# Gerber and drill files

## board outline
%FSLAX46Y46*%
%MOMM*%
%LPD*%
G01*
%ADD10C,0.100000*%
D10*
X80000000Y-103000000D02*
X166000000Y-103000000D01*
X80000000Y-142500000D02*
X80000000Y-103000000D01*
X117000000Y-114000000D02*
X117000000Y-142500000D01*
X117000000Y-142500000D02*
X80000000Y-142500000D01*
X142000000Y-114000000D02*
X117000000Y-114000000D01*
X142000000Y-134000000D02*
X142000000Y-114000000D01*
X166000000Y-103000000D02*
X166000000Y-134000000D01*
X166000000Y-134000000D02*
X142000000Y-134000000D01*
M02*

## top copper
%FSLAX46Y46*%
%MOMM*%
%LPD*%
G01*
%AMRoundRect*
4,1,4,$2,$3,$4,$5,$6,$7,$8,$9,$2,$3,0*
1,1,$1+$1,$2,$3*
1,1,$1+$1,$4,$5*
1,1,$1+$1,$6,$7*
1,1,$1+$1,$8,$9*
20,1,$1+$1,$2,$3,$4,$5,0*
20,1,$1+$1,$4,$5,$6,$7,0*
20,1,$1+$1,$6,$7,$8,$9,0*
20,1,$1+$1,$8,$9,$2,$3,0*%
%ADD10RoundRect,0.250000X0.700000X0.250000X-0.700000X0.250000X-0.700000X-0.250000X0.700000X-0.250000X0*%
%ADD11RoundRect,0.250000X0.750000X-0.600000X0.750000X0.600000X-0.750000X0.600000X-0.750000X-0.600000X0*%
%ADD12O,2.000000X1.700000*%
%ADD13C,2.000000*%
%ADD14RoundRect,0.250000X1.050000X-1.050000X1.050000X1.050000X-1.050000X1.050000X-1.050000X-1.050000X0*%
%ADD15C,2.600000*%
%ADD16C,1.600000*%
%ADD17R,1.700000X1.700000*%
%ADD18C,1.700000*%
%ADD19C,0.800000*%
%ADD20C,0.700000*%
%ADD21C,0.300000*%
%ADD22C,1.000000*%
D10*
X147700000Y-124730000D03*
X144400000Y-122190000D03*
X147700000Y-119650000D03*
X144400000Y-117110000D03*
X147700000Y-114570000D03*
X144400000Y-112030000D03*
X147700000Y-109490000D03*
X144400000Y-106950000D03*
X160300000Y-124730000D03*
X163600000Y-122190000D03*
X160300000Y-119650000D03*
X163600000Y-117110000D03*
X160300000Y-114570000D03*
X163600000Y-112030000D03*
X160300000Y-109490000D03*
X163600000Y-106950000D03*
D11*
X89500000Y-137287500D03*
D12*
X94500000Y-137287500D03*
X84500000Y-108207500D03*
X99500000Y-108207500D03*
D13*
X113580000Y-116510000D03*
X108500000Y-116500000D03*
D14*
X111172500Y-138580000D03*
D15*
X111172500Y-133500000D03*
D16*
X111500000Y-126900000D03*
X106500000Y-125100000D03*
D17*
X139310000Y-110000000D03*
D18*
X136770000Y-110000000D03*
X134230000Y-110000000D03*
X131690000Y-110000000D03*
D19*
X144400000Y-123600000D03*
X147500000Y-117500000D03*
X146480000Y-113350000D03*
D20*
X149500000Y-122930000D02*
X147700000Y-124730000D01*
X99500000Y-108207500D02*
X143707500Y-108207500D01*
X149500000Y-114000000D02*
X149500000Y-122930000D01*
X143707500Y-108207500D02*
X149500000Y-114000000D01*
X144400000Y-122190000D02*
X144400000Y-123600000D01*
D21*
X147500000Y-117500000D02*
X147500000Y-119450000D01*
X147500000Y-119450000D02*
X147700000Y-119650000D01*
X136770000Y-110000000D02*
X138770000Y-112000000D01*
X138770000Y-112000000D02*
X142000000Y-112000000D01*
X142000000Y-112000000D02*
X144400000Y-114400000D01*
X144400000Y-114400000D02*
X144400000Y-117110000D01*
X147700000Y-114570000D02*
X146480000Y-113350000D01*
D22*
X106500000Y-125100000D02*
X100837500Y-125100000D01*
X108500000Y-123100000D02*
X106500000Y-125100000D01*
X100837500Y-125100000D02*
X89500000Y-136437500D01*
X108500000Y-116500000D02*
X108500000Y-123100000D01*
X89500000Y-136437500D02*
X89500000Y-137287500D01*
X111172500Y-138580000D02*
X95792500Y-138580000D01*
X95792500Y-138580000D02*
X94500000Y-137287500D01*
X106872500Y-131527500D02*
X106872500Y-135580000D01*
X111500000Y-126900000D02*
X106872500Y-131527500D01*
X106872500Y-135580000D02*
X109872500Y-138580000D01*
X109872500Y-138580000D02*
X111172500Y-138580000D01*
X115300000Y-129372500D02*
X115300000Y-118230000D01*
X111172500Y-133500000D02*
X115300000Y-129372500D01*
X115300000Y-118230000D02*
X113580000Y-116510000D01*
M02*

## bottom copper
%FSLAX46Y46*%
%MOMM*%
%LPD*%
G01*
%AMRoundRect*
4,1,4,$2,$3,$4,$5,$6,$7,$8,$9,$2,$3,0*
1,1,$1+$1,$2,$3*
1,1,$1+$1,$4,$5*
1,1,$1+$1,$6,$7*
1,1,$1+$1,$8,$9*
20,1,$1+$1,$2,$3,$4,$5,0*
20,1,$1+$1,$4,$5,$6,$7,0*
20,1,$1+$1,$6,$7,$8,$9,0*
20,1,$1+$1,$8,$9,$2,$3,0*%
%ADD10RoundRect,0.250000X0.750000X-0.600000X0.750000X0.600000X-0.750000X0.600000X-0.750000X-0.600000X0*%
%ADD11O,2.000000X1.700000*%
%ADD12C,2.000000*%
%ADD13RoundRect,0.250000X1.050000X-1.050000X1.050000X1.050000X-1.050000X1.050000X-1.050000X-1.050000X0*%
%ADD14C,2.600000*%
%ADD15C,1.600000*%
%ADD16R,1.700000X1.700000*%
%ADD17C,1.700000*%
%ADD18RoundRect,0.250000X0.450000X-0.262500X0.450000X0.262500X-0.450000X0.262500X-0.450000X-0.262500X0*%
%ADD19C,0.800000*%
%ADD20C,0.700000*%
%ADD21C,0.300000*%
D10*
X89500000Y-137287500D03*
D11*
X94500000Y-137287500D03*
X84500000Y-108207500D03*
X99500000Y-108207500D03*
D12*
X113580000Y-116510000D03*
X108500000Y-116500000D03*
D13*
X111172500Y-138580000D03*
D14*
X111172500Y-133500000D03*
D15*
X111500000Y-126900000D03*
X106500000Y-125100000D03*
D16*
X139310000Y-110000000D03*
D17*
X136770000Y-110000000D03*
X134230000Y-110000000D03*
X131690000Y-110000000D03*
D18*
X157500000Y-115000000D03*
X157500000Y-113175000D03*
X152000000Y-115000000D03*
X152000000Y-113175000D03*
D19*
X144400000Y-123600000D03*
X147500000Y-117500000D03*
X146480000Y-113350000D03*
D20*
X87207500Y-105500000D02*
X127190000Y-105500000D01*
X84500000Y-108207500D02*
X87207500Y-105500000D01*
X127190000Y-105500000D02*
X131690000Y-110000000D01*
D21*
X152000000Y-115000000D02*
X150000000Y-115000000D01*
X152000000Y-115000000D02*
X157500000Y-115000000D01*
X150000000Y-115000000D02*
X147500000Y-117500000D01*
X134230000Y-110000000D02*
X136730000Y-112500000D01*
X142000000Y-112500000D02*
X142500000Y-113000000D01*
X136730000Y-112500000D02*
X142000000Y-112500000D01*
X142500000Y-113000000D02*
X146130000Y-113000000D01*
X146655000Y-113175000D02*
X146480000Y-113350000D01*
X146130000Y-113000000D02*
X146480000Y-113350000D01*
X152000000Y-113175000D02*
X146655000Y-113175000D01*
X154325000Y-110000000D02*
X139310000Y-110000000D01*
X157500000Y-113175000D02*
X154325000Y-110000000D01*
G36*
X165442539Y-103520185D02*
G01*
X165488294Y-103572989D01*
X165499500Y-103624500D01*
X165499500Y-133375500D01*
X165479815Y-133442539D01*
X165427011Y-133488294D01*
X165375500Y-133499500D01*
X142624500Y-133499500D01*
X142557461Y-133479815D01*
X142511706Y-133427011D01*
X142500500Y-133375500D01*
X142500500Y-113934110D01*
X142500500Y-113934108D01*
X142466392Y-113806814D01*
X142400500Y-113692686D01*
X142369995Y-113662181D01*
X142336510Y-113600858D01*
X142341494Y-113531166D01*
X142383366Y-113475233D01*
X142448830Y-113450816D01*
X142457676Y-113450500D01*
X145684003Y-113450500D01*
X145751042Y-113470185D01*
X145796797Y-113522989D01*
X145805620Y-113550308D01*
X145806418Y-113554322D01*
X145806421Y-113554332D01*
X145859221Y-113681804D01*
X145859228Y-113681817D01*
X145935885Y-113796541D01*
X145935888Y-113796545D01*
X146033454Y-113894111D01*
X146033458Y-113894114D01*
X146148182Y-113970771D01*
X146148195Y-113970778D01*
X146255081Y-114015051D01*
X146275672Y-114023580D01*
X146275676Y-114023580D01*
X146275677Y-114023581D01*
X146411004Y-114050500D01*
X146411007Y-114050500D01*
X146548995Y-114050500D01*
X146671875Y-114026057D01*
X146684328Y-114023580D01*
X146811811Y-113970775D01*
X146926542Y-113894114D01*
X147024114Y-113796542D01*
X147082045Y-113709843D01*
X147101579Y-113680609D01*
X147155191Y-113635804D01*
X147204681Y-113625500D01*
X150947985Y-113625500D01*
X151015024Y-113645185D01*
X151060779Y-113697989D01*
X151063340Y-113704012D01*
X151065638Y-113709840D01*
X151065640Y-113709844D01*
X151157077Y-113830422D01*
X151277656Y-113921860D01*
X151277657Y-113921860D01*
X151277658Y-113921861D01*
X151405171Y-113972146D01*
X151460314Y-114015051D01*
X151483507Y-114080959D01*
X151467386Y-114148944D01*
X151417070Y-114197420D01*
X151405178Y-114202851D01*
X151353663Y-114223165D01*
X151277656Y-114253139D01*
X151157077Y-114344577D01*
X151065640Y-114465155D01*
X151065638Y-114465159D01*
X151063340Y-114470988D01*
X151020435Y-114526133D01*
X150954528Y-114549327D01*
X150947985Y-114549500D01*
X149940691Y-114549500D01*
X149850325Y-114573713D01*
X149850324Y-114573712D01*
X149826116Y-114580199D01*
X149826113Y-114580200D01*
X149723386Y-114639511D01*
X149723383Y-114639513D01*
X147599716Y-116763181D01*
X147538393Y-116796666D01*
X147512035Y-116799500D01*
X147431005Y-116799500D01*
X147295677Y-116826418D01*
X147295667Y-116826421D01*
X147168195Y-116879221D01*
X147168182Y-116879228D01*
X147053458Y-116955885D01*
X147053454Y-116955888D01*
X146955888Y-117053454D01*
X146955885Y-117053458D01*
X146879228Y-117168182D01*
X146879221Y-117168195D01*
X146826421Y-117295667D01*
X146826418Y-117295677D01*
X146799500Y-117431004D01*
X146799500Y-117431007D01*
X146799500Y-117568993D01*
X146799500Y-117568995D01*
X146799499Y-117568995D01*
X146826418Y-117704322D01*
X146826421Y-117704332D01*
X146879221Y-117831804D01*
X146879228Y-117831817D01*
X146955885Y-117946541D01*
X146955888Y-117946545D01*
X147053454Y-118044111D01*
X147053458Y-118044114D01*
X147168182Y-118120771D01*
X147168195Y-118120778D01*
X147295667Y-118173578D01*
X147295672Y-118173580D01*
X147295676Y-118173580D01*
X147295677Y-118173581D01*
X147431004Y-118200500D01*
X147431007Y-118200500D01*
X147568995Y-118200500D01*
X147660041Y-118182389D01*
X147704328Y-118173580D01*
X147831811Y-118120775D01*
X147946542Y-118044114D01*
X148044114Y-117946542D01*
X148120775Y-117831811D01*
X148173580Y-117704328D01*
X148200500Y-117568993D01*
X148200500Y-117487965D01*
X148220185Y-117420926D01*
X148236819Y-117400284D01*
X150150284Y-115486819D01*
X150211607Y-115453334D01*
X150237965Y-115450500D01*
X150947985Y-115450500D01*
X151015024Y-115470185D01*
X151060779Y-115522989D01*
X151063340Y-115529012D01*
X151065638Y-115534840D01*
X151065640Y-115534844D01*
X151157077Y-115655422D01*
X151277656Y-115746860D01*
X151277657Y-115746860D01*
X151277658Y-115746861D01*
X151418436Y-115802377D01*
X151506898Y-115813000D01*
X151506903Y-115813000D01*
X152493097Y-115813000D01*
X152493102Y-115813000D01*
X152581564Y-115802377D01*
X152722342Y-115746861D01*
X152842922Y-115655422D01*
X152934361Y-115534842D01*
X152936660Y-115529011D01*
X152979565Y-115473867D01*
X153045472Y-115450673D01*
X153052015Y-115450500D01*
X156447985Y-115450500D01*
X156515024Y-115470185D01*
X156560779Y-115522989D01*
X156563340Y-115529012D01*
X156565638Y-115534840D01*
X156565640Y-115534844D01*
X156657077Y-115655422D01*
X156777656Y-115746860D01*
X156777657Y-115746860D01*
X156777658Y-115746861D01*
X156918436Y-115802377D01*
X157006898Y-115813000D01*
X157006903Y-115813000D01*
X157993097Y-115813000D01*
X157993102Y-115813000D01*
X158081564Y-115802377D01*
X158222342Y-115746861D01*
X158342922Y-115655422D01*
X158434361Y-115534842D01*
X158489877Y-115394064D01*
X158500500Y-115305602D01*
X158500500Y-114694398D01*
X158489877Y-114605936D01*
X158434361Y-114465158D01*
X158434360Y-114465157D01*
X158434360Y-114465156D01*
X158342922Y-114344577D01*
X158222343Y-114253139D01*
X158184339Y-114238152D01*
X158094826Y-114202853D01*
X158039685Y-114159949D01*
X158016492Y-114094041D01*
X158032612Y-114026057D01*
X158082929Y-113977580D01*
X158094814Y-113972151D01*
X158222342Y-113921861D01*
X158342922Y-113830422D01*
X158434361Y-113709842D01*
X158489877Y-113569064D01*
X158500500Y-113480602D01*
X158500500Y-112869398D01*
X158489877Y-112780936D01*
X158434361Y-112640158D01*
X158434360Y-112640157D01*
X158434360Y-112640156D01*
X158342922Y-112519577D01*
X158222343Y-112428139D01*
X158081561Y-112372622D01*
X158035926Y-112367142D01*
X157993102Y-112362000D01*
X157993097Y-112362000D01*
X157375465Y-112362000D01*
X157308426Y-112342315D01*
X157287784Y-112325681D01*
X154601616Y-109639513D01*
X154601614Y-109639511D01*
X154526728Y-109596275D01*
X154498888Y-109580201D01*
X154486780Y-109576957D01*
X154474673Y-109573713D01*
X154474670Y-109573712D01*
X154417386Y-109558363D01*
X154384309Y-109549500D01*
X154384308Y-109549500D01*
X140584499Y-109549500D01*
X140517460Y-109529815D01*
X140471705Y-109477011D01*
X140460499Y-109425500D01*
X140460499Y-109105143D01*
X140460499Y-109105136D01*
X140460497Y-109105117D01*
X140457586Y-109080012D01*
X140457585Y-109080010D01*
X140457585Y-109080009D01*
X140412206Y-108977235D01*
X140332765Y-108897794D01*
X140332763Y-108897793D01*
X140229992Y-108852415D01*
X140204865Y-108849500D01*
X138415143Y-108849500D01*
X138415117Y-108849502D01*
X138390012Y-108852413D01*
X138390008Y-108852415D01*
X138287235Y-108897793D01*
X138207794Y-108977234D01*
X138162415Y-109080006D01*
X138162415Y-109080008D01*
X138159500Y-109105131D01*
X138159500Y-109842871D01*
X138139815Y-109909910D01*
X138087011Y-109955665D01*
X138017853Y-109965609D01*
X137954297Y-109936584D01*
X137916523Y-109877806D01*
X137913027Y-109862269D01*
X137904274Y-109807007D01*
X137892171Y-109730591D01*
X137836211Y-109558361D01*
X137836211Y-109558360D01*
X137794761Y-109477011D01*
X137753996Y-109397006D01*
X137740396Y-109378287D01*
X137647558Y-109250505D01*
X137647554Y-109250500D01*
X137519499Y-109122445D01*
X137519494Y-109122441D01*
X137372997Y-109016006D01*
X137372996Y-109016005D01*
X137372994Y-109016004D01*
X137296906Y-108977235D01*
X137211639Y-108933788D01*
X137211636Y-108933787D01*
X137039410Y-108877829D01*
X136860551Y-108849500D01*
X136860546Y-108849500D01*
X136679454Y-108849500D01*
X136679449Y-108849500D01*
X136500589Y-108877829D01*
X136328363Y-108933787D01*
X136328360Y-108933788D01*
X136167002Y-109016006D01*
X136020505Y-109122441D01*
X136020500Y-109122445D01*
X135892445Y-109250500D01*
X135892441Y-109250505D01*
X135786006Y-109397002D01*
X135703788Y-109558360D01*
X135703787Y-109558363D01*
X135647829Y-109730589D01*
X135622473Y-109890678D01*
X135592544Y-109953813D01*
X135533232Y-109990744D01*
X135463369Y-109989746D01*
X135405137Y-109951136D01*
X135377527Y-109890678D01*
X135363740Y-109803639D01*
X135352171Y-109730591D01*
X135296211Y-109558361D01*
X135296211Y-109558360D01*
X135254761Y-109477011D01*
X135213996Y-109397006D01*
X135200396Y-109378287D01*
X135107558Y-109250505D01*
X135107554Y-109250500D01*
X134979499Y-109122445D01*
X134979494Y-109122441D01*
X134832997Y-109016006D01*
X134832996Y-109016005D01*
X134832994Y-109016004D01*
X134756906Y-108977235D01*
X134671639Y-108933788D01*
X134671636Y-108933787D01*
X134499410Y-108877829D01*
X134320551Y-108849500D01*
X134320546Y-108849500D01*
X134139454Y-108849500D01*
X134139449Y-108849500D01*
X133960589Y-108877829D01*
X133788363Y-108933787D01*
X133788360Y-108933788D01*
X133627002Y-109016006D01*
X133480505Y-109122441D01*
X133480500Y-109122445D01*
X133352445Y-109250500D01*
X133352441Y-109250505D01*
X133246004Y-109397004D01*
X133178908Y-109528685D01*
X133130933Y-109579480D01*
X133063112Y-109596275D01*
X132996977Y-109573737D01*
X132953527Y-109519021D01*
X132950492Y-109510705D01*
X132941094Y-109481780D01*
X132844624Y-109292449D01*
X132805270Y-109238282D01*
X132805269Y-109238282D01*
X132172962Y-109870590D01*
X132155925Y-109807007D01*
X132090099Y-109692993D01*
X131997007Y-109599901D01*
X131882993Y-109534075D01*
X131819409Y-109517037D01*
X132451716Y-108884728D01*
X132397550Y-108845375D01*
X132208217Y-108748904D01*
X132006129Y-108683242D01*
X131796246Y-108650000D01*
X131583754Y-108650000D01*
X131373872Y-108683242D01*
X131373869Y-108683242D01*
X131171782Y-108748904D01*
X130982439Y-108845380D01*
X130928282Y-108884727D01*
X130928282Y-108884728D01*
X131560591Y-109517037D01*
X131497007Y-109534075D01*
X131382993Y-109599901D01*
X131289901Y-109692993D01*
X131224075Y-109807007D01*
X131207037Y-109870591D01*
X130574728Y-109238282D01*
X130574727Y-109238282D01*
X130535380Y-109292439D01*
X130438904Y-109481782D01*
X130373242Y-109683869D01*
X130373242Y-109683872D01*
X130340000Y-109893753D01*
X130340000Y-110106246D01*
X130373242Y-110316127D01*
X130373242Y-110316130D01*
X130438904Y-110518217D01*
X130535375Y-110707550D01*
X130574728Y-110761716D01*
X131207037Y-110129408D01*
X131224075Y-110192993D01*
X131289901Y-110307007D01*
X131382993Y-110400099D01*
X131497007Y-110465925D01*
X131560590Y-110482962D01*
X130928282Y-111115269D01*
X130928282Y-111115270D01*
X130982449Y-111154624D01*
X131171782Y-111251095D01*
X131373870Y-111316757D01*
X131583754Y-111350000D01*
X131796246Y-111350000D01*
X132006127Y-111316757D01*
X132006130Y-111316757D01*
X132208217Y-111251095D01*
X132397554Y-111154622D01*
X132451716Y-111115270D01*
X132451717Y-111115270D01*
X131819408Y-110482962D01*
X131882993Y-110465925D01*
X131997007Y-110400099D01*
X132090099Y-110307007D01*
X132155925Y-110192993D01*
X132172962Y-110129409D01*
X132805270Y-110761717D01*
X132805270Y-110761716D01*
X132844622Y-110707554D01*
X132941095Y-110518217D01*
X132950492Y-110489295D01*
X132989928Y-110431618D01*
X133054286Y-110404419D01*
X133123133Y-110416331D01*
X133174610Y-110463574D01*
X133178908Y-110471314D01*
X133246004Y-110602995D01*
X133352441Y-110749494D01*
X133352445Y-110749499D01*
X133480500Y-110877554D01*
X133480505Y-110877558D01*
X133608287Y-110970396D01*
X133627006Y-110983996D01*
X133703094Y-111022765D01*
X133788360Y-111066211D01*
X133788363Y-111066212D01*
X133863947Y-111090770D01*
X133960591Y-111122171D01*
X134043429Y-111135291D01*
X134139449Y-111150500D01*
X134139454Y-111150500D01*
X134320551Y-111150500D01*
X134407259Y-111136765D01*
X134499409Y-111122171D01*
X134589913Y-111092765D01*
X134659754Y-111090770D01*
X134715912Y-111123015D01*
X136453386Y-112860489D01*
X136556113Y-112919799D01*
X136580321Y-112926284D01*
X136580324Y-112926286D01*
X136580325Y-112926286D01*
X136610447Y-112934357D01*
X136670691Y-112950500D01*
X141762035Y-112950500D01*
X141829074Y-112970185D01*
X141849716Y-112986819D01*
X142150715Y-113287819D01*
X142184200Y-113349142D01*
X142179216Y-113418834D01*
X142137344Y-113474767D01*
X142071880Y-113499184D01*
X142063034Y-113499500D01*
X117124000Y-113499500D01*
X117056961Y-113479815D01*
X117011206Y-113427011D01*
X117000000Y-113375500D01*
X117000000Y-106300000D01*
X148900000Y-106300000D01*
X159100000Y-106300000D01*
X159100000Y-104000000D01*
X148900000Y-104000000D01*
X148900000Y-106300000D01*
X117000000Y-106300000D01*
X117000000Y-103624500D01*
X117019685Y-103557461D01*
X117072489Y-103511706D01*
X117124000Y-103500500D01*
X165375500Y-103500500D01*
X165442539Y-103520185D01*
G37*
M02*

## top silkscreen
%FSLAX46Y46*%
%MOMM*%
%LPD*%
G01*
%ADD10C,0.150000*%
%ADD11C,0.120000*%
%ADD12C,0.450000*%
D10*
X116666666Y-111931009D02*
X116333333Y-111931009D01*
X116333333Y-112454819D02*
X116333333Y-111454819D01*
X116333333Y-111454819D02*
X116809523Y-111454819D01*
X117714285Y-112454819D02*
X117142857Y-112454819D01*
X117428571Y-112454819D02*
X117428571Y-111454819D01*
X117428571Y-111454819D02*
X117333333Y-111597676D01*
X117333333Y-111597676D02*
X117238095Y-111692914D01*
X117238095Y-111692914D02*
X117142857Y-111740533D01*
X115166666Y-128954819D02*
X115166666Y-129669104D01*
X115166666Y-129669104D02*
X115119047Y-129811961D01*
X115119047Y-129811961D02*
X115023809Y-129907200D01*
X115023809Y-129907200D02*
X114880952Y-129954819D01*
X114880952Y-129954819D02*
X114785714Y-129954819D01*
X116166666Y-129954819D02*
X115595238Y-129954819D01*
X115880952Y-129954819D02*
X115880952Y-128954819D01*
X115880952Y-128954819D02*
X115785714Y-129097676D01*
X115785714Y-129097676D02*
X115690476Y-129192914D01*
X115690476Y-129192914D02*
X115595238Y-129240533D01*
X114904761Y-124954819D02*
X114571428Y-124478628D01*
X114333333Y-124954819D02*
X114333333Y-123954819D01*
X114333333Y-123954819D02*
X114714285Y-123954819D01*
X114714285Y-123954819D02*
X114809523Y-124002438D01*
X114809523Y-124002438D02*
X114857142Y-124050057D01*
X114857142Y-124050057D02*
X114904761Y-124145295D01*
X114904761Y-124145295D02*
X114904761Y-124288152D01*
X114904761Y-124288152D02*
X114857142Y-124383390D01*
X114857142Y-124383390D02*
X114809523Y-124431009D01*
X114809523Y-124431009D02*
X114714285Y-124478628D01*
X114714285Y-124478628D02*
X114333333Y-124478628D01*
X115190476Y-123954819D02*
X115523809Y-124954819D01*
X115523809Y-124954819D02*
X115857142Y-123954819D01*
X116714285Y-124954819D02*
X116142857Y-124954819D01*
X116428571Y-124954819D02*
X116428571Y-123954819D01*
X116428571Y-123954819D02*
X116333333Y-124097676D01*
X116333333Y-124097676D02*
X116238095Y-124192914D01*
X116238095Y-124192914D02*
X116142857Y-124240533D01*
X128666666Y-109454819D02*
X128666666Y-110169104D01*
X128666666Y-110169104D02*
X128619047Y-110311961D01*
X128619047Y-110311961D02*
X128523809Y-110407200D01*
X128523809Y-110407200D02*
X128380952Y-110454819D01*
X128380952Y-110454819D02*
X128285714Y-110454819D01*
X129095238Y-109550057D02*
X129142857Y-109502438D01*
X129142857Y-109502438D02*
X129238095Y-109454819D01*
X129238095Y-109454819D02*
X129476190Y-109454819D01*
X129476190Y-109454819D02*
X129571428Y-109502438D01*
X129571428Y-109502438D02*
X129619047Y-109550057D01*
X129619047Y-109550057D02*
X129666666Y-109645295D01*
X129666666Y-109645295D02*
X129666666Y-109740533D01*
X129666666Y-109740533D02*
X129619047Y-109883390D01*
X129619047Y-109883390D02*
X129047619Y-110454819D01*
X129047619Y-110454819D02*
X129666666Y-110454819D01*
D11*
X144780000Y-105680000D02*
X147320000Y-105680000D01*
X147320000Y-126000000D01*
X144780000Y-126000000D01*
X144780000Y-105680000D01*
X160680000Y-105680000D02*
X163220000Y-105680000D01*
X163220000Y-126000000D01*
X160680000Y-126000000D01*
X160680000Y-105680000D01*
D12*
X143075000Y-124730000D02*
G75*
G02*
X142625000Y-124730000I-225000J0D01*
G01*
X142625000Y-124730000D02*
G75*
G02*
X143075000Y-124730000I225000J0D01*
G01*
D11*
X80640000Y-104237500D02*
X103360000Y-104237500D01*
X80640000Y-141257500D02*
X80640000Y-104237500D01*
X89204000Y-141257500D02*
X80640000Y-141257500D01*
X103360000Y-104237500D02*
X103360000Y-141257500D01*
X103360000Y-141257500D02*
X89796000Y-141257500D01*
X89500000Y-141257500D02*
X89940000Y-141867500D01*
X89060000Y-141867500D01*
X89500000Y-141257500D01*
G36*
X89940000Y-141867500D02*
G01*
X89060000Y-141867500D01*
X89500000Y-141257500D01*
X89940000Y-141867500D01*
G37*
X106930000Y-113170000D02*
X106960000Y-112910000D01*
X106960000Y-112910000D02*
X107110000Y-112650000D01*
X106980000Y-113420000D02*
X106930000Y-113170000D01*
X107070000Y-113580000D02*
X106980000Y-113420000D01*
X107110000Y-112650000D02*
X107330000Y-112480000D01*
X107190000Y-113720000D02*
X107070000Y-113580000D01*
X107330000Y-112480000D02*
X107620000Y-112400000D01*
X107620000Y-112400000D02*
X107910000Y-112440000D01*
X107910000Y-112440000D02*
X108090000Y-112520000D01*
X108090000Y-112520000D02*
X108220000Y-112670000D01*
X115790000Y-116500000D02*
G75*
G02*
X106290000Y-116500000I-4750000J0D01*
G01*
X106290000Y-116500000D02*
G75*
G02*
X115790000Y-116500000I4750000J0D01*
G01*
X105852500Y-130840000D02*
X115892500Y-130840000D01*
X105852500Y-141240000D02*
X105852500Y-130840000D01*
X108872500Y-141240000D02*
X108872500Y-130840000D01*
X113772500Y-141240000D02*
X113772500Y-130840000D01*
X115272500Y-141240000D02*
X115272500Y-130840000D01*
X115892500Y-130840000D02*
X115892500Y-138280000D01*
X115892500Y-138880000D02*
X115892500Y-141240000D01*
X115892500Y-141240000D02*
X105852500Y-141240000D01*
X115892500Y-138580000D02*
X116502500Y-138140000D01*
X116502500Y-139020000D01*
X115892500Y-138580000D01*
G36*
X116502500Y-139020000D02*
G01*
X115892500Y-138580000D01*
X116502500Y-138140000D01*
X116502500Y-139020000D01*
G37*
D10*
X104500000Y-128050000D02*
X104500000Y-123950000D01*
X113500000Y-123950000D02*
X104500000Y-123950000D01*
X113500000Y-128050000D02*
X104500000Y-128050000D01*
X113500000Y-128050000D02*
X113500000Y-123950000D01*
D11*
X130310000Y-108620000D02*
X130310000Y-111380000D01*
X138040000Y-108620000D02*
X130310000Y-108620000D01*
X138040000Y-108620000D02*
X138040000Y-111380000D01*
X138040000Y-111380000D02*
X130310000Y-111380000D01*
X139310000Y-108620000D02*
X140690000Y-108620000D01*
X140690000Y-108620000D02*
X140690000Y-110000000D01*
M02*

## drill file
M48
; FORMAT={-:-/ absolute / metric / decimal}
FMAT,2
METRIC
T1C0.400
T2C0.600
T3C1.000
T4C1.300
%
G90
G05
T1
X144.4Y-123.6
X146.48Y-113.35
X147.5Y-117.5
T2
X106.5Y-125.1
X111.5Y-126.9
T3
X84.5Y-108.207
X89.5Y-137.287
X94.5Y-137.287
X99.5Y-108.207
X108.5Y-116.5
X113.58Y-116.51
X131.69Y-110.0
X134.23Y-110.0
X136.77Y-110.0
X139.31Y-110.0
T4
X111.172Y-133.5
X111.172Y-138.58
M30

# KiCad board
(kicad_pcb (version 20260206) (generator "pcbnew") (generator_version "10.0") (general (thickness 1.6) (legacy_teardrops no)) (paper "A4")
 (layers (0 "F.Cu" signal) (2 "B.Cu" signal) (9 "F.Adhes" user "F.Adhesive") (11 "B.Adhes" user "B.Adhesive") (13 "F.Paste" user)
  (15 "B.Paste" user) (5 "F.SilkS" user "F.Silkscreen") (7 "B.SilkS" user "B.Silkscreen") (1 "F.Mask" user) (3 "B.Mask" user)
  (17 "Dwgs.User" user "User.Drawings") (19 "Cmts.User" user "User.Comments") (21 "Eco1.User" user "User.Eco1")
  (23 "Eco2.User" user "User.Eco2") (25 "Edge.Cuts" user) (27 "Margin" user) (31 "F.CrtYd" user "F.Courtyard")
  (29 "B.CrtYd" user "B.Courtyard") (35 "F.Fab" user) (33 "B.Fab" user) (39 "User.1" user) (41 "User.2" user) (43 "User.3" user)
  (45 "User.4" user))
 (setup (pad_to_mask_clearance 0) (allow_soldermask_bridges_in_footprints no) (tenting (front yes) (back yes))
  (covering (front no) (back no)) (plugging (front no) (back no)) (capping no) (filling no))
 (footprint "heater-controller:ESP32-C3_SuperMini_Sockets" (layer "F.Cu") (at 154 115 180)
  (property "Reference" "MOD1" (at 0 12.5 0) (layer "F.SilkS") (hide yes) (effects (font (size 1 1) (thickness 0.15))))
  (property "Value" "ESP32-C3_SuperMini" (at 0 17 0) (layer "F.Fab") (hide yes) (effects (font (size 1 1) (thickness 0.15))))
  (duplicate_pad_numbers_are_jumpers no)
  (fp_rect (start 6.68 -11) (end 9.22 9.32) (stroke (width 0.12) (type solid)) (fill no) (layer "F.SilkS"))
  (fp_rect (start -9.22 -11) (end -6.68 9.32) (stroke (width 0.12) (type solid)) (fill no) (layer "F.SilkS"))
  (fp_circle (center 11.15 -9.73) (end 11.45 -9.73) (stroke (width 0.3) (type solid)) (fill yes) (layer "F.SilkS"))
  (pad "1" smd roundrect (at 6.3 -9.73 180) (size 1.9 1) (layers "F.Cu" "F.Mask" "F.Paste") (roundrect_rratio 0.25) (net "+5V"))
  (pad "2" smd roundrect (at 9.6 -7.19 180) (size 1.9 1) (layers "F.Cu" "F.Mask" "F.Paste") (roundrect_rratio 0.25) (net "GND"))
  (pad "3" smd roundrect (at 6.3 -4.65 180) (size 1.9 1) (layers "F.Cu" "F.Mask" "F.Paste") (roundrect_rratio 0.25) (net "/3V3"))
  (pad "4" smd roundrect (at 9.6 -2.11 180) (size 1.9 1) (layers "F.Cu" "F.Mask" "F.Paste") (roundrect_rratio 0.25) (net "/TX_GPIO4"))
  (pad "5" smd roundrect (at 6.3 0.43 180) (size 1.9 1) (layers "F.Cu" "F.Mask" "F.Paste") (roundrect_rratio 0.25) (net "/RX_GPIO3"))
  (pad "6" smd roundrect (at 9.6 2.97 180) (size 1.9 1) (layers "F.Cu" "F.Mask" "F.Paste") (roundrect_rratio 0.25)
   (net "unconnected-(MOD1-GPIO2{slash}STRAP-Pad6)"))
  (pad "7" smd roundrect (at 6.3 5.51 180) (size 1.9 1) (layers "F.Cu" "F.Mask" "F.Paste") (roundrect_rratio 0.25)
   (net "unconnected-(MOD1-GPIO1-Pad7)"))
  (pad "8" smd roundrect (at 9.6 8.05 180) (size 1.9 1) (layers "F.Cu" "F.Mask" "F.Paste") (roundrect_rratio 0.25)
   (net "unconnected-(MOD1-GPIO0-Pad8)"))
  (pad "9" smd roundrect (at -6.3 -9.73 180) (size 1.9 1) (layers "F.Cu" "F.Mask" "F.Paste") (roundrect_rratio 0.25)
   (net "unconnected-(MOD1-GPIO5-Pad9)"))
  (pad "10" smd roundrect (at -9.6 -7.19 180) (size 1.9 1) (layers "F.Cu" "F.Mask" "F.Paste") (roundrect_rratio 0.25)
   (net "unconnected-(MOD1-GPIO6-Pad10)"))
  (pad "11" smd roundrect (at -6.3 -4.65 180) (size 1.9 1) (layers "F.Cu" "F.Mask" "F.Paste") (roundrect_rratio 0.25)
   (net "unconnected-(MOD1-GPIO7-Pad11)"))
  (pad "12" smd roundrect (at -9.6 -2.11 180) (size 1.9 1) (layers "F.Cu" "F.Mask" "F.Paste") (roundrect_rratio 0.25)
   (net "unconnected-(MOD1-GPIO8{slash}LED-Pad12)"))
  (pad "13" smd roundrect (at -6.3 0.43 180) (size 1.9 1) (layers "F.Cu" "F.Mask" "F.Paste") (roundrect_rratio 0.25)
   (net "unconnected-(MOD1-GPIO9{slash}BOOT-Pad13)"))
  (pad "14" smd roundrect (at -9.6 2.97 180) (size 1.9 1) (layers "F.Cu" "F.Mask" "F.Paste") (roundrect_rratio 0.25)
   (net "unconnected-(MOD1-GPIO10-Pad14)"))
  (pad "15" smd roundrect (at -6.3 5.51 180) (size 1.9 1) (layers "F.Cu" "F.Mask" "F.Paste") (roundrect_rratio 0.25)
   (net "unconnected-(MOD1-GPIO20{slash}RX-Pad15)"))
  (pad "16" smd roundrect (at -9.6 8.05 180) (size 1.9 1) (layers "F.Cu" "F.Mask" "F.Paste") (roundrect_rratio 0.25)
   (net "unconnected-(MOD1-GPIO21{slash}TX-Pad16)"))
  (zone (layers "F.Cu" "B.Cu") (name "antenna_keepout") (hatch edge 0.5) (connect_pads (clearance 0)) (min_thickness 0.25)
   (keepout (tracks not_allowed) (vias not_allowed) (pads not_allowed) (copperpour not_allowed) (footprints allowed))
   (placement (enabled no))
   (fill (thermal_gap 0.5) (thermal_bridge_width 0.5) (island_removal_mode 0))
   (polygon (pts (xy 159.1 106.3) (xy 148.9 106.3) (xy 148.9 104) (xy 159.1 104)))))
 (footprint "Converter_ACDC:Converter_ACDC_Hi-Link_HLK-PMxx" (layer "F.Cu") (at 89.5 137.2875 90)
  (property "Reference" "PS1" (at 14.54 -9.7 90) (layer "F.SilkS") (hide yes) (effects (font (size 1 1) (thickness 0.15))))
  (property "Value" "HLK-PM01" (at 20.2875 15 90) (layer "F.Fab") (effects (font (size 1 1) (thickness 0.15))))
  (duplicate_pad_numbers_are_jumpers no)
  (fp_line (start 33.05 -8.86) (end 33.05 13.86) (stroke (width 0.12) (type solid)) (layer "F.SilkS"))
  (fp_line (start -3.97 -8.86) (end 33.05 -8.86) (stroke (width 0.12) (type solid)) (layer "F.SilkS"))
  (fp_line (start -3.97 -0.296) (end -3.97 -8.86) (stroke (width 0.12) (type solid)) (layer "F.SilkS"))
  (fp_line (start 33.05 13.86) (end -3.97 13.86) (stroke (width 0.12) (type solid)) (layer "F.SilkS"))
  (fp_line (start -3.97 13.86) (end -3.97 0.296) (stroke (width 0.12) (type solid)) (layer "F.SilkS"))
  (fp_poly (pts (xy -3.97 0) (xy -4.58 0.44) (xy -4.58 -0.44)) (stroke (width 0.12) (type solid)) (fill yes) (layer "F.SilkS"))
  (pad "1" thru_hole roundrect (at 0 0 90) (size 1.7 2) (drill 1) (layers "*.Cu" "*.Mask") (remove_unused_layers no)
   (roundrect_rratio 0.147059) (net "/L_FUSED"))
  (pad "2" thru_hole oval (at 0 5 90) (size 1.7 2) (drill 1) (layers "*.Cu" "*.Mask") (remove_unused_layers no) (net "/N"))
  (pad "3" thru_hole oval (at 29.08 -5 90) (size 1.7 2) (drill 1) (layers "*.Cu" "*.Mask") (remove_unused_layers no) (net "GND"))
  (pad "4" thru_hole oval (at 29.08 10 90) (size 1.7 2) (drill 1) (layers "*.Cu" "*.Mask") (remove_unused_layers no) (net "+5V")))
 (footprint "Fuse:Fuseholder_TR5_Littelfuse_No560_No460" (layer "F.Cu") (at 113.58 116.51 180)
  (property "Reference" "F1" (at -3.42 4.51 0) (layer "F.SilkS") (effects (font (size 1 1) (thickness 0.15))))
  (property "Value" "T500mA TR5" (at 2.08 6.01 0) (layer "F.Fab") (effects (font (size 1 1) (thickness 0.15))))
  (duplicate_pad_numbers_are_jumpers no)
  (fp_line (start 6.65 3.34) (end 6.62 3.6) (stroke (width 0.12) (type solid)) (layer "F.SilkS"))
  (fp_line (start 6.62 3.6) (end 6.47 3.86) (stroke (width 0.12) (type solid)) (layer "F.SilkS"))
  (fp_line (start 6.6 3.09) (end 6.65 3.34) (stroke (width 0.12) (type solid)) (layer "F.SilkS"))
  (fp_line (start 6.51 2.93) (end 6.6 3.09) (stroke (width 0.12) (type solid)) (layer "F.SilkS"))
  (fp_line (start 6.47 3.86) (end 6.25 4.03) (stroke (width 0.12) (type solid)) (layer "F.SilkS"))
  (fp_line (start 6.39 2.79) (end 6.51 2.93) (stroke (width 0.12) (type solid)) (layer "F.SilkS"))
  (fp_line (start 6.25 4.03) (end 5.96 4.11) (stroke (width 0.12) (type solid)) (layer "F.SilkS"))
  (fp_line (start 5.96 4.11) (end 5.67 4.07) (stroke (width 0.12) (type solid)) (layer "F.SilkS"))
  (fp_line (start 5.67 4.07) (end 5.49 3.99) (stroke (width 0.12) (type solid)) (layer "F.SilkS"))
  (fp_line (start 5.49 3.99) (end 5.36 3.84) (stroke (width 0.12) (type solid)) (layer "F.SilkS"))
  (fp_circle (center 2.54 0.01) (end 7.29 0.01) (stroke (width 0.12) (type solid)) (fill no) (layer "F.SilkS"))
  (pad "1" thru_hole circle (at 0 0 180) (size 2 2) (drill 1) (layers "*.Cu" "*.Mask") (remove_unused_layers no) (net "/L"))
  (pad "2" thru_hole circle (at 5.08 0.01 180) (size 2 2) (drill 1) (layers "*.Cu" "*.Mask") (remove_unused_layers no) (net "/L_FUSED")))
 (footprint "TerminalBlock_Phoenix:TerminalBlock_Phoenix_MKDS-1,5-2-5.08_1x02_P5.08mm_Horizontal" (layer "F.Cu") (at 111.1725 138.58 90)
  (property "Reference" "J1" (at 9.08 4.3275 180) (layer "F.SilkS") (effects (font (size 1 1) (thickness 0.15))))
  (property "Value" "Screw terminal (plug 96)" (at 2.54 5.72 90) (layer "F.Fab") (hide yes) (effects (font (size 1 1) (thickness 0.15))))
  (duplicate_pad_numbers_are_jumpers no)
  (fp_line (start 7.74 -5.32) (end 7.74 4.72) (stroke (width 0.12) (type solid)) (layer "F.SilkS"))
  (fp_line (start -2.66 -5.32) (end 7.74 -5.32) (stroke (width 0.12) (type solid)) (layer "F.SilkS"))
  (fp_line (start -2.66 -2.3) (end 7.74 -2.3) (stroke (width 0.12) (type solid)) (layer "F.SilkS"))
  (fp_line (start -2.66 2.6) (end 7.74 2.6) (stroke (width 0.12) (type solid)) (layer "F.SilkS"))
  (fp_line (start -2.66 4.1) (end 7.74 4.1) (stroke (width 0.12) (type solid)) (layer "F.SilkS"))
  (fp_line (start 7.74 4.72) (end 0.3 4.72) (stroke (width 0.12) (type solid)) (layer "F.SilkS"))
  (fp_line (start -0.3 4.72) (end -2.66 4.72) (stroke (width 0.12) (type solid)) (layer "F.SilkS"))
  (fp_line (start -2.66 4.72) (end -2.66 -5.32) (stroke (width 0.12) (type solid)) (layer "F.SilkS"))
  (fp_poly (pts (xy 0 4.72) (xy 0.44 5.33) (xy -0.44 5.33)) (stroke (width 0.12) (type solid)) (fill yes) (layer "F.SilkS"))
  (pad "1" thru_hole roundrect (at 0 0 90) (size 2.6 2.6) (drill 1.3) (layers "*.Cu" "*.Mask") (remove_unused_layers no)
   (roundrect_rratio 0.096154) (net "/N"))
  (pad "2" thru_hole circle (at 5.08 0 90) (size 2.6 2.6) (drill 1.3) (layers "*.Cu" "*.Mask") (remove_unused_layers no) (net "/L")))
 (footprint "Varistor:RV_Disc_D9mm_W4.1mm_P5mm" (layer "F.Cu") (at 111.5 126.9 180)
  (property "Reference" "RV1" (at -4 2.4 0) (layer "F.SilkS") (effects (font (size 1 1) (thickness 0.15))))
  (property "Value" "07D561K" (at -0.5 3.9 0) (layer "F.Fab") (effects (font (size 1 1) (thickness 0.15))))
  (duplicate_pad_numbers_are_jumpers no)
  (fp_line (start 7 -1.15) (end 7 2.95) (stroke (width 0.15) (type solid)) (layer "F.SilkS"))
  (fp_line (start -2 2.95) (end 7 2.95) (stroke (width 0.15) (type solid)) (layer "F.SilkS"))
  (fp_line (start -2 -1.15) (end 7 -1.15) (stroke (width 0.15) (type solid)) (layer "F.SilkS"))
  (fp_line (start -2 -1.15) (end -2 2.95) (stroke (width 0.15) (type solid)) (layer "F.SilkS"))
  (pad "1" thru_hole circle (at 0 0 180) (size 1.6 1.6) (drill 0.6) (layers "*.Cu" "*.Mask") (remove_unused_layers no) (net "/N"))
  (pad "2" thru_hole circle (at 5 1.8 180) (size 1.6 1.6) (drill 0.6) (layers "*.Cu" "*.Mask") (remove_unused_layers no) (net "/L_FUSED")))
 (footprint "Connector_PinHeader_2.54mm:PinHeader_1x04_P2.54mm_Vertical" (layer "F.Cu") (at 139.31 110 -90)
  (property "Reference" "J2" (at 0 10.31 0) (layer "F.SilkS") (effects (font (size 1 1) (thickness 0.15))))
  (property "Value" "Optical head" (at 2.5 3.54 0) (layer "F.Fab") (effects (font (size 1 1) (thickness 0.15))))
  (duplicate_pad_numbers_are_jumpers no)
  (fp_line (start -1.38 9) (end 1.38 9) (stroke (width 0.12) (type solid)) (layer "F.SilkS"))
  (fp_line (start -1.38 1.27) (end -1.38 9) (stroke (width 0.12) (type solid)) (layer "F.SilkS"))
  (fp_line (start -1.38 1.27) (end 1.38 1.27) (stroke (width 0.12) (type solid)) (layer "F.SilkS"))
  (fp_line (start 1.38 1.27) (end 1.38 9) (stroke (width 0.12) (type solid)) (layer "F.SilkS"))
  (fp_line (start -1.38 0) (end -1.38 -1.38) (stroke (width 0.12) (type solid)) (layer "F.SilkS"))
  (fp_line (start -1.38 -1.38) (end 0 -1.38) (stroke (width 0.12) (type solid)) (layer "F.SilkS"))
  (pad "1" thru_hole rect (at 0 0 270) (size 1.7 1.7) (drill 1) (layers "*.Cu" "*.Mask") (remove_unused_layers no) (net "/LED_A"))
  (pad "2" thru_hole circle (at 0 2.54 270) (size 1.7 1.7) (drill 1) (layers "*.Cu" "*.Mask") (remove_unused_layers no) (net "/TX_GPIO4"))
  (pad "3" thru_hole circle (at 0 5.08 270) (size 1.7 1.7) (drill 1) (layers "*.Cu" "*.Mask") (remove_unused_layers no) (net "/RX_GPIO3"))
  (pad "4" thru_hole circle (at 0 7.62 270) (size 1.7 1.7) (drill 1) (layers "*.Cu" "*.Mask") (remove_unused_layers no) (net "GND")))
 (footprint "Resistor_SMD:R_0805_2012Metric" (layer "B.Cu") (at 157.5 114.0875 90)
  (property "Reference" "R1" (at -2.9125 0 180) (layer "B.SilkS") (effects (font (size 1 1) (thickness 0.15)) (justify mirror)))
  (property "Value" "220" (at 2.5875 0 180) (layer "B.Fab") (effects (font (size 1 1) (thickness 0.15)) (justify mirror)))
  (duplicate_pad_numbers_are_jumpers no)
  (pad "1" smd roundrect (at -0.9125 0 90) (size 1.025 1.4) (layers "B.Cu" "B.Mask" "B.Paste") (roundrect_rratio 0.243902) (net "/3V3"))
  (pad "2" smd roundrect (at 0.9125 0 90) (size 1.025 1.4) (layers "B.Cu" "B.Mask" "B.Paste") (roundrect_rratio 0.243902) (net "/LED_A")))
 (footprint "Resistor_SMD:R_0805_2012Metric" (layer "B.Cu") (at 152 114.0875 90)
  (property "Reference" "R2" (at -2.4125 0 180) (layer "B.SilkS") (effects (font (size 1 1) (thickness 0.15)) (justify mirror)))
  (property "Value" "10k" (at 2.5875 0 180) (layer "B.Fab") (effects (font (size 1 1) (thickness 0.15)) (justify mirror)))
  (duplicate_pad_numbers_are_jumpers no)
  (pad "1" smd roundrect (at -0.9125 0 90) (size 1.025 1.4) (layers "B.Cu" "B.Mask" "B.Paste") (roundrect_rratio 0.243902) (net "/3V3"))
  (pad "2" smd roundrect (at 0.9125 0 90) (size 1.025 1.4) (layers "B.Cu" "B.Mask" "B.Paste") (roundrect_rratio 0.243902) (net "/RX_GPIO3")))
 (gr_line (start 80 103) (end 166 103) (stroke (width 0.1) (type default)) (layer "Edge.Cuts"))
 (gr_line (start 80 142.5) (end 80 103) (stroke (width 0.1) (type default)) (layer "Edge.Cuts"))
 (gr_line (start 117 114) (end 117 142.5) (stroke (width 0.1) (type default)) (layer "Edge.Cuts"))
 (gr_line (start 117 142.5) (end 80 142.5) (stroke (width 0.1) (type default)) (layer "Edge.Cuts"))
 (gr_line (start 142 114) (end 117 114) (stroke (width 0.1) (type default)) (layer "Edge.Cuts"))
 (gr_line (start 142 134) (end 142 114) (stroke (width 0.1) (type default)) (layer "Edge.Cuts"))
 (gr_line (start 166 103) (end 166 134) (stroke (width 0.1) (type default)) (layer "Edge.Cuts"))
 (gr_line (start 166 134) (end 142 134) (stroke (width 0.1) (type default)) (layer "Edge.Cuts"))
 (segment (start 149.5 122.93) (end 147.7 124.73) (width 0.7) (layer "F.Cu") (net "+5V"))
 (segment (start 99.5 108.2075) (end 143.7075 108.2075) (width 0.7) (layer "F.Cu") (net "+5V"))
 (segment (start 149.5 114) (end 149.5 122.93) (width 0.7) (layer "F.Cu") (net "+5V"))
 (segment (start 143.7075 108.2075) (end 149.5 114) (width 0.7) (layer "F.Cu") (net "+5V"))
 (segment (start 144.4 122.19) (end 144.4 123.6) (width 0.7) (layer "F.Cu") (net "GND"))
 (via (at 144.4 123.6) (size 0.8) (drill 0.4) (layers "F.Cu" "B.Cu") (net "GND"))
 (segment (start 87.2075 105.5) (end 127.19 105.5) (width 0.7) (layer "B.Cu") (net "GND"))
 (segment (start 84.5 108.2075) (end 87.2075 105.5) (width 0.7) (layer "B.Cu") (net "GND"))
 (segment (start 127.19 105.5) (end 131.69 110) (width 0.7) (layer "B.Cu") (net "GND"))
 (segment (start 147.5 117.5) (end 147.5 119.45) (width 0.3) (layer "F.Cu") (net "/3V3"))
 (segment (start 147.5 119.45) (end 147.7 119.65) (width 0.3) (layer "F.Cu") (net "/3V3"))
 (via (at 147.5 117.5) (size 0.8) (drill 0.4) (layers "F.Cu" "B.Cu") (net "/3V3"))
 (segment (start 152 115) (end 150 115) (width 0.3) (layer "B.Cu") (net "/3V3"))
 (segment (start 152 115) (end 157.5 115) (width 0.3) (layer "B.Cu") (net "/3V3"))
 (segment (start 150 115) (end 147.5 117.5) (width 0.3) (layer "B.Cu") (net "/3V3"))
 (segment (start 136.77 110) (end 138.77 112) (width 0.3) (layer "F.Cu") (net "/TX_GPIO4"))
 (segment (start 138.77 112) (end 142 112) (width 0.3) (layer "F.Cu") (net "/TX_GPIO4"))
 (segment (start 142 112) (end 144.4 114.4) (width 0.3) (layer "F.Cu") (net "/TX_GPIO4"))
 (segment (start 144.4 114.4) (end 144.4 117.11) (width 0.3) (layer "F.Cu") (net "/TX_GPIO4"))
 (segment (start 147.7 114.57) (end 146.48 113.35) (width 0.3) (layer "F.Cu") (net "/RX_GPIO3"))
 (via (at 146.48 113.35) (size 0.8) (drill 0.4) (layers "F.Cu" "B.Cu") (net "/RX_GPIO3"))
 (segment (start 134.23 110) (end 136.73 112.5) (width 0.3) (layer "B.Cu") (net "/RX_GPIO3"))
 (segment (start 142 112.5) (end 142.5 113) (width 0.3) (layer "B.Cu") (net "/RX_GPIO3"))
 (segment (start 136.73 112.5) (end 142 112.5) (width 0.3) (layer "B.Cu") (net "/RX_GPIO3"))
 (segment (start 142.5 113) (end 146.13 113) (width 0.3) (layer "B.Cu") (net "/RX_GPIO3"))
 (segment (start 146.655 113.175) (end 146.48 113.35) (width 0.3) (layer "B.Cu") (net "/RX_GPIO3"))
 (segment (start 146.13 113) (end 146.48 113.35) (width 0.3) (layer "B.Cu") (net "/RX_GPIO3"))
 (segment (start 152 113.175) (end 146.655 113.175) (width 0.3) (layer "B.Cu") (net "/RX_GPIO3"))
 (segment (start 106.5 125.1) (end 100.8375 125.1) (width 1) (layer "F.Cu") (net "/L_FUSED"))
 (segment (start 108.5 123.1) (end 106.5 125.1) (width 1) (layer "F.Cu") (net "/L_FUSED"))
 (segment (start 100.8375 125.1) (end 89.5 136.4375) (width 1) (layer "F.Cu") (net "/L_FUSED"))
 (segment (start 108.5 116.5) (end 108.5 123.1) (width 1) (layer "F.Cu") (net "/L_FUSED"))
 (segment (start 89.5 136.4375) (end 89.5 137.2875) (width 1) (layer "F.Cu") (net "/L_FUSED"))
 (segment (start 111.1725 138.58) (end 95.7925 138.58) (width 1) (layer "F.Cu") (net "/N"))
 (segment (start 95.7925 138.58) (end 94.5 137.2875) (width 1) (layer "F.Cu") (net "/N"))
 (segment (start 106.8725 131.5275) (end 106.8725 135.58) (width 1) (layer "F.Cu") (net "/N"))
 (segment (start 111.5 126.9) (end 106.8725 131.5275) (width 1) (layer "F.Cu") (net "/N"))
 (segment (start 106.8725 135.58) (end 109.8725 138.58) (width 1) (layer "F.Cu") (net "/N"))
 (segment (start 109.8725 138.58) (end 111.1725 138.58) (width 1) (layer "F.Cu") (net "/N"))
 (segment (start 115.3 129.3725) (end 115.3 118.23) (width 1) (layer "F.Cu") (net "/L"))
 (segment (start 111.1725 133.5) (end 115.3 129.3725) (width 1) (layer "F.Cu") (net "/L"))
 (segment (start 115.3 118.23) (end 113.58 116.51) (width 1) (layer "F.Cu") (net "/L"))
 (segment (start 154.325 110) (end 139.31 110) (width 0.3) (layer "B.Cu") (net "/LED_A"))
 (segment (start 157.5 113.175) (end 154.325 110) (width 0.3) (layer "B.Cu") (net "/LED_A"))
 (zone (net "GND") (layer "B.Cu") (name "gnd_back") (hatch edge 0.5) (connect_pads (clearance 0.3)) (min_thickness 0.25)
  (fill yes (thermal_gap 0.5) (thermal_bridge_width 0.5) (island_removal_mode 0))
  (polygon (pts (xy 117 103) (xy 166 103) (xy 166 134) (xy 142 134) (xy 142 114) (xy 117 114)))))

